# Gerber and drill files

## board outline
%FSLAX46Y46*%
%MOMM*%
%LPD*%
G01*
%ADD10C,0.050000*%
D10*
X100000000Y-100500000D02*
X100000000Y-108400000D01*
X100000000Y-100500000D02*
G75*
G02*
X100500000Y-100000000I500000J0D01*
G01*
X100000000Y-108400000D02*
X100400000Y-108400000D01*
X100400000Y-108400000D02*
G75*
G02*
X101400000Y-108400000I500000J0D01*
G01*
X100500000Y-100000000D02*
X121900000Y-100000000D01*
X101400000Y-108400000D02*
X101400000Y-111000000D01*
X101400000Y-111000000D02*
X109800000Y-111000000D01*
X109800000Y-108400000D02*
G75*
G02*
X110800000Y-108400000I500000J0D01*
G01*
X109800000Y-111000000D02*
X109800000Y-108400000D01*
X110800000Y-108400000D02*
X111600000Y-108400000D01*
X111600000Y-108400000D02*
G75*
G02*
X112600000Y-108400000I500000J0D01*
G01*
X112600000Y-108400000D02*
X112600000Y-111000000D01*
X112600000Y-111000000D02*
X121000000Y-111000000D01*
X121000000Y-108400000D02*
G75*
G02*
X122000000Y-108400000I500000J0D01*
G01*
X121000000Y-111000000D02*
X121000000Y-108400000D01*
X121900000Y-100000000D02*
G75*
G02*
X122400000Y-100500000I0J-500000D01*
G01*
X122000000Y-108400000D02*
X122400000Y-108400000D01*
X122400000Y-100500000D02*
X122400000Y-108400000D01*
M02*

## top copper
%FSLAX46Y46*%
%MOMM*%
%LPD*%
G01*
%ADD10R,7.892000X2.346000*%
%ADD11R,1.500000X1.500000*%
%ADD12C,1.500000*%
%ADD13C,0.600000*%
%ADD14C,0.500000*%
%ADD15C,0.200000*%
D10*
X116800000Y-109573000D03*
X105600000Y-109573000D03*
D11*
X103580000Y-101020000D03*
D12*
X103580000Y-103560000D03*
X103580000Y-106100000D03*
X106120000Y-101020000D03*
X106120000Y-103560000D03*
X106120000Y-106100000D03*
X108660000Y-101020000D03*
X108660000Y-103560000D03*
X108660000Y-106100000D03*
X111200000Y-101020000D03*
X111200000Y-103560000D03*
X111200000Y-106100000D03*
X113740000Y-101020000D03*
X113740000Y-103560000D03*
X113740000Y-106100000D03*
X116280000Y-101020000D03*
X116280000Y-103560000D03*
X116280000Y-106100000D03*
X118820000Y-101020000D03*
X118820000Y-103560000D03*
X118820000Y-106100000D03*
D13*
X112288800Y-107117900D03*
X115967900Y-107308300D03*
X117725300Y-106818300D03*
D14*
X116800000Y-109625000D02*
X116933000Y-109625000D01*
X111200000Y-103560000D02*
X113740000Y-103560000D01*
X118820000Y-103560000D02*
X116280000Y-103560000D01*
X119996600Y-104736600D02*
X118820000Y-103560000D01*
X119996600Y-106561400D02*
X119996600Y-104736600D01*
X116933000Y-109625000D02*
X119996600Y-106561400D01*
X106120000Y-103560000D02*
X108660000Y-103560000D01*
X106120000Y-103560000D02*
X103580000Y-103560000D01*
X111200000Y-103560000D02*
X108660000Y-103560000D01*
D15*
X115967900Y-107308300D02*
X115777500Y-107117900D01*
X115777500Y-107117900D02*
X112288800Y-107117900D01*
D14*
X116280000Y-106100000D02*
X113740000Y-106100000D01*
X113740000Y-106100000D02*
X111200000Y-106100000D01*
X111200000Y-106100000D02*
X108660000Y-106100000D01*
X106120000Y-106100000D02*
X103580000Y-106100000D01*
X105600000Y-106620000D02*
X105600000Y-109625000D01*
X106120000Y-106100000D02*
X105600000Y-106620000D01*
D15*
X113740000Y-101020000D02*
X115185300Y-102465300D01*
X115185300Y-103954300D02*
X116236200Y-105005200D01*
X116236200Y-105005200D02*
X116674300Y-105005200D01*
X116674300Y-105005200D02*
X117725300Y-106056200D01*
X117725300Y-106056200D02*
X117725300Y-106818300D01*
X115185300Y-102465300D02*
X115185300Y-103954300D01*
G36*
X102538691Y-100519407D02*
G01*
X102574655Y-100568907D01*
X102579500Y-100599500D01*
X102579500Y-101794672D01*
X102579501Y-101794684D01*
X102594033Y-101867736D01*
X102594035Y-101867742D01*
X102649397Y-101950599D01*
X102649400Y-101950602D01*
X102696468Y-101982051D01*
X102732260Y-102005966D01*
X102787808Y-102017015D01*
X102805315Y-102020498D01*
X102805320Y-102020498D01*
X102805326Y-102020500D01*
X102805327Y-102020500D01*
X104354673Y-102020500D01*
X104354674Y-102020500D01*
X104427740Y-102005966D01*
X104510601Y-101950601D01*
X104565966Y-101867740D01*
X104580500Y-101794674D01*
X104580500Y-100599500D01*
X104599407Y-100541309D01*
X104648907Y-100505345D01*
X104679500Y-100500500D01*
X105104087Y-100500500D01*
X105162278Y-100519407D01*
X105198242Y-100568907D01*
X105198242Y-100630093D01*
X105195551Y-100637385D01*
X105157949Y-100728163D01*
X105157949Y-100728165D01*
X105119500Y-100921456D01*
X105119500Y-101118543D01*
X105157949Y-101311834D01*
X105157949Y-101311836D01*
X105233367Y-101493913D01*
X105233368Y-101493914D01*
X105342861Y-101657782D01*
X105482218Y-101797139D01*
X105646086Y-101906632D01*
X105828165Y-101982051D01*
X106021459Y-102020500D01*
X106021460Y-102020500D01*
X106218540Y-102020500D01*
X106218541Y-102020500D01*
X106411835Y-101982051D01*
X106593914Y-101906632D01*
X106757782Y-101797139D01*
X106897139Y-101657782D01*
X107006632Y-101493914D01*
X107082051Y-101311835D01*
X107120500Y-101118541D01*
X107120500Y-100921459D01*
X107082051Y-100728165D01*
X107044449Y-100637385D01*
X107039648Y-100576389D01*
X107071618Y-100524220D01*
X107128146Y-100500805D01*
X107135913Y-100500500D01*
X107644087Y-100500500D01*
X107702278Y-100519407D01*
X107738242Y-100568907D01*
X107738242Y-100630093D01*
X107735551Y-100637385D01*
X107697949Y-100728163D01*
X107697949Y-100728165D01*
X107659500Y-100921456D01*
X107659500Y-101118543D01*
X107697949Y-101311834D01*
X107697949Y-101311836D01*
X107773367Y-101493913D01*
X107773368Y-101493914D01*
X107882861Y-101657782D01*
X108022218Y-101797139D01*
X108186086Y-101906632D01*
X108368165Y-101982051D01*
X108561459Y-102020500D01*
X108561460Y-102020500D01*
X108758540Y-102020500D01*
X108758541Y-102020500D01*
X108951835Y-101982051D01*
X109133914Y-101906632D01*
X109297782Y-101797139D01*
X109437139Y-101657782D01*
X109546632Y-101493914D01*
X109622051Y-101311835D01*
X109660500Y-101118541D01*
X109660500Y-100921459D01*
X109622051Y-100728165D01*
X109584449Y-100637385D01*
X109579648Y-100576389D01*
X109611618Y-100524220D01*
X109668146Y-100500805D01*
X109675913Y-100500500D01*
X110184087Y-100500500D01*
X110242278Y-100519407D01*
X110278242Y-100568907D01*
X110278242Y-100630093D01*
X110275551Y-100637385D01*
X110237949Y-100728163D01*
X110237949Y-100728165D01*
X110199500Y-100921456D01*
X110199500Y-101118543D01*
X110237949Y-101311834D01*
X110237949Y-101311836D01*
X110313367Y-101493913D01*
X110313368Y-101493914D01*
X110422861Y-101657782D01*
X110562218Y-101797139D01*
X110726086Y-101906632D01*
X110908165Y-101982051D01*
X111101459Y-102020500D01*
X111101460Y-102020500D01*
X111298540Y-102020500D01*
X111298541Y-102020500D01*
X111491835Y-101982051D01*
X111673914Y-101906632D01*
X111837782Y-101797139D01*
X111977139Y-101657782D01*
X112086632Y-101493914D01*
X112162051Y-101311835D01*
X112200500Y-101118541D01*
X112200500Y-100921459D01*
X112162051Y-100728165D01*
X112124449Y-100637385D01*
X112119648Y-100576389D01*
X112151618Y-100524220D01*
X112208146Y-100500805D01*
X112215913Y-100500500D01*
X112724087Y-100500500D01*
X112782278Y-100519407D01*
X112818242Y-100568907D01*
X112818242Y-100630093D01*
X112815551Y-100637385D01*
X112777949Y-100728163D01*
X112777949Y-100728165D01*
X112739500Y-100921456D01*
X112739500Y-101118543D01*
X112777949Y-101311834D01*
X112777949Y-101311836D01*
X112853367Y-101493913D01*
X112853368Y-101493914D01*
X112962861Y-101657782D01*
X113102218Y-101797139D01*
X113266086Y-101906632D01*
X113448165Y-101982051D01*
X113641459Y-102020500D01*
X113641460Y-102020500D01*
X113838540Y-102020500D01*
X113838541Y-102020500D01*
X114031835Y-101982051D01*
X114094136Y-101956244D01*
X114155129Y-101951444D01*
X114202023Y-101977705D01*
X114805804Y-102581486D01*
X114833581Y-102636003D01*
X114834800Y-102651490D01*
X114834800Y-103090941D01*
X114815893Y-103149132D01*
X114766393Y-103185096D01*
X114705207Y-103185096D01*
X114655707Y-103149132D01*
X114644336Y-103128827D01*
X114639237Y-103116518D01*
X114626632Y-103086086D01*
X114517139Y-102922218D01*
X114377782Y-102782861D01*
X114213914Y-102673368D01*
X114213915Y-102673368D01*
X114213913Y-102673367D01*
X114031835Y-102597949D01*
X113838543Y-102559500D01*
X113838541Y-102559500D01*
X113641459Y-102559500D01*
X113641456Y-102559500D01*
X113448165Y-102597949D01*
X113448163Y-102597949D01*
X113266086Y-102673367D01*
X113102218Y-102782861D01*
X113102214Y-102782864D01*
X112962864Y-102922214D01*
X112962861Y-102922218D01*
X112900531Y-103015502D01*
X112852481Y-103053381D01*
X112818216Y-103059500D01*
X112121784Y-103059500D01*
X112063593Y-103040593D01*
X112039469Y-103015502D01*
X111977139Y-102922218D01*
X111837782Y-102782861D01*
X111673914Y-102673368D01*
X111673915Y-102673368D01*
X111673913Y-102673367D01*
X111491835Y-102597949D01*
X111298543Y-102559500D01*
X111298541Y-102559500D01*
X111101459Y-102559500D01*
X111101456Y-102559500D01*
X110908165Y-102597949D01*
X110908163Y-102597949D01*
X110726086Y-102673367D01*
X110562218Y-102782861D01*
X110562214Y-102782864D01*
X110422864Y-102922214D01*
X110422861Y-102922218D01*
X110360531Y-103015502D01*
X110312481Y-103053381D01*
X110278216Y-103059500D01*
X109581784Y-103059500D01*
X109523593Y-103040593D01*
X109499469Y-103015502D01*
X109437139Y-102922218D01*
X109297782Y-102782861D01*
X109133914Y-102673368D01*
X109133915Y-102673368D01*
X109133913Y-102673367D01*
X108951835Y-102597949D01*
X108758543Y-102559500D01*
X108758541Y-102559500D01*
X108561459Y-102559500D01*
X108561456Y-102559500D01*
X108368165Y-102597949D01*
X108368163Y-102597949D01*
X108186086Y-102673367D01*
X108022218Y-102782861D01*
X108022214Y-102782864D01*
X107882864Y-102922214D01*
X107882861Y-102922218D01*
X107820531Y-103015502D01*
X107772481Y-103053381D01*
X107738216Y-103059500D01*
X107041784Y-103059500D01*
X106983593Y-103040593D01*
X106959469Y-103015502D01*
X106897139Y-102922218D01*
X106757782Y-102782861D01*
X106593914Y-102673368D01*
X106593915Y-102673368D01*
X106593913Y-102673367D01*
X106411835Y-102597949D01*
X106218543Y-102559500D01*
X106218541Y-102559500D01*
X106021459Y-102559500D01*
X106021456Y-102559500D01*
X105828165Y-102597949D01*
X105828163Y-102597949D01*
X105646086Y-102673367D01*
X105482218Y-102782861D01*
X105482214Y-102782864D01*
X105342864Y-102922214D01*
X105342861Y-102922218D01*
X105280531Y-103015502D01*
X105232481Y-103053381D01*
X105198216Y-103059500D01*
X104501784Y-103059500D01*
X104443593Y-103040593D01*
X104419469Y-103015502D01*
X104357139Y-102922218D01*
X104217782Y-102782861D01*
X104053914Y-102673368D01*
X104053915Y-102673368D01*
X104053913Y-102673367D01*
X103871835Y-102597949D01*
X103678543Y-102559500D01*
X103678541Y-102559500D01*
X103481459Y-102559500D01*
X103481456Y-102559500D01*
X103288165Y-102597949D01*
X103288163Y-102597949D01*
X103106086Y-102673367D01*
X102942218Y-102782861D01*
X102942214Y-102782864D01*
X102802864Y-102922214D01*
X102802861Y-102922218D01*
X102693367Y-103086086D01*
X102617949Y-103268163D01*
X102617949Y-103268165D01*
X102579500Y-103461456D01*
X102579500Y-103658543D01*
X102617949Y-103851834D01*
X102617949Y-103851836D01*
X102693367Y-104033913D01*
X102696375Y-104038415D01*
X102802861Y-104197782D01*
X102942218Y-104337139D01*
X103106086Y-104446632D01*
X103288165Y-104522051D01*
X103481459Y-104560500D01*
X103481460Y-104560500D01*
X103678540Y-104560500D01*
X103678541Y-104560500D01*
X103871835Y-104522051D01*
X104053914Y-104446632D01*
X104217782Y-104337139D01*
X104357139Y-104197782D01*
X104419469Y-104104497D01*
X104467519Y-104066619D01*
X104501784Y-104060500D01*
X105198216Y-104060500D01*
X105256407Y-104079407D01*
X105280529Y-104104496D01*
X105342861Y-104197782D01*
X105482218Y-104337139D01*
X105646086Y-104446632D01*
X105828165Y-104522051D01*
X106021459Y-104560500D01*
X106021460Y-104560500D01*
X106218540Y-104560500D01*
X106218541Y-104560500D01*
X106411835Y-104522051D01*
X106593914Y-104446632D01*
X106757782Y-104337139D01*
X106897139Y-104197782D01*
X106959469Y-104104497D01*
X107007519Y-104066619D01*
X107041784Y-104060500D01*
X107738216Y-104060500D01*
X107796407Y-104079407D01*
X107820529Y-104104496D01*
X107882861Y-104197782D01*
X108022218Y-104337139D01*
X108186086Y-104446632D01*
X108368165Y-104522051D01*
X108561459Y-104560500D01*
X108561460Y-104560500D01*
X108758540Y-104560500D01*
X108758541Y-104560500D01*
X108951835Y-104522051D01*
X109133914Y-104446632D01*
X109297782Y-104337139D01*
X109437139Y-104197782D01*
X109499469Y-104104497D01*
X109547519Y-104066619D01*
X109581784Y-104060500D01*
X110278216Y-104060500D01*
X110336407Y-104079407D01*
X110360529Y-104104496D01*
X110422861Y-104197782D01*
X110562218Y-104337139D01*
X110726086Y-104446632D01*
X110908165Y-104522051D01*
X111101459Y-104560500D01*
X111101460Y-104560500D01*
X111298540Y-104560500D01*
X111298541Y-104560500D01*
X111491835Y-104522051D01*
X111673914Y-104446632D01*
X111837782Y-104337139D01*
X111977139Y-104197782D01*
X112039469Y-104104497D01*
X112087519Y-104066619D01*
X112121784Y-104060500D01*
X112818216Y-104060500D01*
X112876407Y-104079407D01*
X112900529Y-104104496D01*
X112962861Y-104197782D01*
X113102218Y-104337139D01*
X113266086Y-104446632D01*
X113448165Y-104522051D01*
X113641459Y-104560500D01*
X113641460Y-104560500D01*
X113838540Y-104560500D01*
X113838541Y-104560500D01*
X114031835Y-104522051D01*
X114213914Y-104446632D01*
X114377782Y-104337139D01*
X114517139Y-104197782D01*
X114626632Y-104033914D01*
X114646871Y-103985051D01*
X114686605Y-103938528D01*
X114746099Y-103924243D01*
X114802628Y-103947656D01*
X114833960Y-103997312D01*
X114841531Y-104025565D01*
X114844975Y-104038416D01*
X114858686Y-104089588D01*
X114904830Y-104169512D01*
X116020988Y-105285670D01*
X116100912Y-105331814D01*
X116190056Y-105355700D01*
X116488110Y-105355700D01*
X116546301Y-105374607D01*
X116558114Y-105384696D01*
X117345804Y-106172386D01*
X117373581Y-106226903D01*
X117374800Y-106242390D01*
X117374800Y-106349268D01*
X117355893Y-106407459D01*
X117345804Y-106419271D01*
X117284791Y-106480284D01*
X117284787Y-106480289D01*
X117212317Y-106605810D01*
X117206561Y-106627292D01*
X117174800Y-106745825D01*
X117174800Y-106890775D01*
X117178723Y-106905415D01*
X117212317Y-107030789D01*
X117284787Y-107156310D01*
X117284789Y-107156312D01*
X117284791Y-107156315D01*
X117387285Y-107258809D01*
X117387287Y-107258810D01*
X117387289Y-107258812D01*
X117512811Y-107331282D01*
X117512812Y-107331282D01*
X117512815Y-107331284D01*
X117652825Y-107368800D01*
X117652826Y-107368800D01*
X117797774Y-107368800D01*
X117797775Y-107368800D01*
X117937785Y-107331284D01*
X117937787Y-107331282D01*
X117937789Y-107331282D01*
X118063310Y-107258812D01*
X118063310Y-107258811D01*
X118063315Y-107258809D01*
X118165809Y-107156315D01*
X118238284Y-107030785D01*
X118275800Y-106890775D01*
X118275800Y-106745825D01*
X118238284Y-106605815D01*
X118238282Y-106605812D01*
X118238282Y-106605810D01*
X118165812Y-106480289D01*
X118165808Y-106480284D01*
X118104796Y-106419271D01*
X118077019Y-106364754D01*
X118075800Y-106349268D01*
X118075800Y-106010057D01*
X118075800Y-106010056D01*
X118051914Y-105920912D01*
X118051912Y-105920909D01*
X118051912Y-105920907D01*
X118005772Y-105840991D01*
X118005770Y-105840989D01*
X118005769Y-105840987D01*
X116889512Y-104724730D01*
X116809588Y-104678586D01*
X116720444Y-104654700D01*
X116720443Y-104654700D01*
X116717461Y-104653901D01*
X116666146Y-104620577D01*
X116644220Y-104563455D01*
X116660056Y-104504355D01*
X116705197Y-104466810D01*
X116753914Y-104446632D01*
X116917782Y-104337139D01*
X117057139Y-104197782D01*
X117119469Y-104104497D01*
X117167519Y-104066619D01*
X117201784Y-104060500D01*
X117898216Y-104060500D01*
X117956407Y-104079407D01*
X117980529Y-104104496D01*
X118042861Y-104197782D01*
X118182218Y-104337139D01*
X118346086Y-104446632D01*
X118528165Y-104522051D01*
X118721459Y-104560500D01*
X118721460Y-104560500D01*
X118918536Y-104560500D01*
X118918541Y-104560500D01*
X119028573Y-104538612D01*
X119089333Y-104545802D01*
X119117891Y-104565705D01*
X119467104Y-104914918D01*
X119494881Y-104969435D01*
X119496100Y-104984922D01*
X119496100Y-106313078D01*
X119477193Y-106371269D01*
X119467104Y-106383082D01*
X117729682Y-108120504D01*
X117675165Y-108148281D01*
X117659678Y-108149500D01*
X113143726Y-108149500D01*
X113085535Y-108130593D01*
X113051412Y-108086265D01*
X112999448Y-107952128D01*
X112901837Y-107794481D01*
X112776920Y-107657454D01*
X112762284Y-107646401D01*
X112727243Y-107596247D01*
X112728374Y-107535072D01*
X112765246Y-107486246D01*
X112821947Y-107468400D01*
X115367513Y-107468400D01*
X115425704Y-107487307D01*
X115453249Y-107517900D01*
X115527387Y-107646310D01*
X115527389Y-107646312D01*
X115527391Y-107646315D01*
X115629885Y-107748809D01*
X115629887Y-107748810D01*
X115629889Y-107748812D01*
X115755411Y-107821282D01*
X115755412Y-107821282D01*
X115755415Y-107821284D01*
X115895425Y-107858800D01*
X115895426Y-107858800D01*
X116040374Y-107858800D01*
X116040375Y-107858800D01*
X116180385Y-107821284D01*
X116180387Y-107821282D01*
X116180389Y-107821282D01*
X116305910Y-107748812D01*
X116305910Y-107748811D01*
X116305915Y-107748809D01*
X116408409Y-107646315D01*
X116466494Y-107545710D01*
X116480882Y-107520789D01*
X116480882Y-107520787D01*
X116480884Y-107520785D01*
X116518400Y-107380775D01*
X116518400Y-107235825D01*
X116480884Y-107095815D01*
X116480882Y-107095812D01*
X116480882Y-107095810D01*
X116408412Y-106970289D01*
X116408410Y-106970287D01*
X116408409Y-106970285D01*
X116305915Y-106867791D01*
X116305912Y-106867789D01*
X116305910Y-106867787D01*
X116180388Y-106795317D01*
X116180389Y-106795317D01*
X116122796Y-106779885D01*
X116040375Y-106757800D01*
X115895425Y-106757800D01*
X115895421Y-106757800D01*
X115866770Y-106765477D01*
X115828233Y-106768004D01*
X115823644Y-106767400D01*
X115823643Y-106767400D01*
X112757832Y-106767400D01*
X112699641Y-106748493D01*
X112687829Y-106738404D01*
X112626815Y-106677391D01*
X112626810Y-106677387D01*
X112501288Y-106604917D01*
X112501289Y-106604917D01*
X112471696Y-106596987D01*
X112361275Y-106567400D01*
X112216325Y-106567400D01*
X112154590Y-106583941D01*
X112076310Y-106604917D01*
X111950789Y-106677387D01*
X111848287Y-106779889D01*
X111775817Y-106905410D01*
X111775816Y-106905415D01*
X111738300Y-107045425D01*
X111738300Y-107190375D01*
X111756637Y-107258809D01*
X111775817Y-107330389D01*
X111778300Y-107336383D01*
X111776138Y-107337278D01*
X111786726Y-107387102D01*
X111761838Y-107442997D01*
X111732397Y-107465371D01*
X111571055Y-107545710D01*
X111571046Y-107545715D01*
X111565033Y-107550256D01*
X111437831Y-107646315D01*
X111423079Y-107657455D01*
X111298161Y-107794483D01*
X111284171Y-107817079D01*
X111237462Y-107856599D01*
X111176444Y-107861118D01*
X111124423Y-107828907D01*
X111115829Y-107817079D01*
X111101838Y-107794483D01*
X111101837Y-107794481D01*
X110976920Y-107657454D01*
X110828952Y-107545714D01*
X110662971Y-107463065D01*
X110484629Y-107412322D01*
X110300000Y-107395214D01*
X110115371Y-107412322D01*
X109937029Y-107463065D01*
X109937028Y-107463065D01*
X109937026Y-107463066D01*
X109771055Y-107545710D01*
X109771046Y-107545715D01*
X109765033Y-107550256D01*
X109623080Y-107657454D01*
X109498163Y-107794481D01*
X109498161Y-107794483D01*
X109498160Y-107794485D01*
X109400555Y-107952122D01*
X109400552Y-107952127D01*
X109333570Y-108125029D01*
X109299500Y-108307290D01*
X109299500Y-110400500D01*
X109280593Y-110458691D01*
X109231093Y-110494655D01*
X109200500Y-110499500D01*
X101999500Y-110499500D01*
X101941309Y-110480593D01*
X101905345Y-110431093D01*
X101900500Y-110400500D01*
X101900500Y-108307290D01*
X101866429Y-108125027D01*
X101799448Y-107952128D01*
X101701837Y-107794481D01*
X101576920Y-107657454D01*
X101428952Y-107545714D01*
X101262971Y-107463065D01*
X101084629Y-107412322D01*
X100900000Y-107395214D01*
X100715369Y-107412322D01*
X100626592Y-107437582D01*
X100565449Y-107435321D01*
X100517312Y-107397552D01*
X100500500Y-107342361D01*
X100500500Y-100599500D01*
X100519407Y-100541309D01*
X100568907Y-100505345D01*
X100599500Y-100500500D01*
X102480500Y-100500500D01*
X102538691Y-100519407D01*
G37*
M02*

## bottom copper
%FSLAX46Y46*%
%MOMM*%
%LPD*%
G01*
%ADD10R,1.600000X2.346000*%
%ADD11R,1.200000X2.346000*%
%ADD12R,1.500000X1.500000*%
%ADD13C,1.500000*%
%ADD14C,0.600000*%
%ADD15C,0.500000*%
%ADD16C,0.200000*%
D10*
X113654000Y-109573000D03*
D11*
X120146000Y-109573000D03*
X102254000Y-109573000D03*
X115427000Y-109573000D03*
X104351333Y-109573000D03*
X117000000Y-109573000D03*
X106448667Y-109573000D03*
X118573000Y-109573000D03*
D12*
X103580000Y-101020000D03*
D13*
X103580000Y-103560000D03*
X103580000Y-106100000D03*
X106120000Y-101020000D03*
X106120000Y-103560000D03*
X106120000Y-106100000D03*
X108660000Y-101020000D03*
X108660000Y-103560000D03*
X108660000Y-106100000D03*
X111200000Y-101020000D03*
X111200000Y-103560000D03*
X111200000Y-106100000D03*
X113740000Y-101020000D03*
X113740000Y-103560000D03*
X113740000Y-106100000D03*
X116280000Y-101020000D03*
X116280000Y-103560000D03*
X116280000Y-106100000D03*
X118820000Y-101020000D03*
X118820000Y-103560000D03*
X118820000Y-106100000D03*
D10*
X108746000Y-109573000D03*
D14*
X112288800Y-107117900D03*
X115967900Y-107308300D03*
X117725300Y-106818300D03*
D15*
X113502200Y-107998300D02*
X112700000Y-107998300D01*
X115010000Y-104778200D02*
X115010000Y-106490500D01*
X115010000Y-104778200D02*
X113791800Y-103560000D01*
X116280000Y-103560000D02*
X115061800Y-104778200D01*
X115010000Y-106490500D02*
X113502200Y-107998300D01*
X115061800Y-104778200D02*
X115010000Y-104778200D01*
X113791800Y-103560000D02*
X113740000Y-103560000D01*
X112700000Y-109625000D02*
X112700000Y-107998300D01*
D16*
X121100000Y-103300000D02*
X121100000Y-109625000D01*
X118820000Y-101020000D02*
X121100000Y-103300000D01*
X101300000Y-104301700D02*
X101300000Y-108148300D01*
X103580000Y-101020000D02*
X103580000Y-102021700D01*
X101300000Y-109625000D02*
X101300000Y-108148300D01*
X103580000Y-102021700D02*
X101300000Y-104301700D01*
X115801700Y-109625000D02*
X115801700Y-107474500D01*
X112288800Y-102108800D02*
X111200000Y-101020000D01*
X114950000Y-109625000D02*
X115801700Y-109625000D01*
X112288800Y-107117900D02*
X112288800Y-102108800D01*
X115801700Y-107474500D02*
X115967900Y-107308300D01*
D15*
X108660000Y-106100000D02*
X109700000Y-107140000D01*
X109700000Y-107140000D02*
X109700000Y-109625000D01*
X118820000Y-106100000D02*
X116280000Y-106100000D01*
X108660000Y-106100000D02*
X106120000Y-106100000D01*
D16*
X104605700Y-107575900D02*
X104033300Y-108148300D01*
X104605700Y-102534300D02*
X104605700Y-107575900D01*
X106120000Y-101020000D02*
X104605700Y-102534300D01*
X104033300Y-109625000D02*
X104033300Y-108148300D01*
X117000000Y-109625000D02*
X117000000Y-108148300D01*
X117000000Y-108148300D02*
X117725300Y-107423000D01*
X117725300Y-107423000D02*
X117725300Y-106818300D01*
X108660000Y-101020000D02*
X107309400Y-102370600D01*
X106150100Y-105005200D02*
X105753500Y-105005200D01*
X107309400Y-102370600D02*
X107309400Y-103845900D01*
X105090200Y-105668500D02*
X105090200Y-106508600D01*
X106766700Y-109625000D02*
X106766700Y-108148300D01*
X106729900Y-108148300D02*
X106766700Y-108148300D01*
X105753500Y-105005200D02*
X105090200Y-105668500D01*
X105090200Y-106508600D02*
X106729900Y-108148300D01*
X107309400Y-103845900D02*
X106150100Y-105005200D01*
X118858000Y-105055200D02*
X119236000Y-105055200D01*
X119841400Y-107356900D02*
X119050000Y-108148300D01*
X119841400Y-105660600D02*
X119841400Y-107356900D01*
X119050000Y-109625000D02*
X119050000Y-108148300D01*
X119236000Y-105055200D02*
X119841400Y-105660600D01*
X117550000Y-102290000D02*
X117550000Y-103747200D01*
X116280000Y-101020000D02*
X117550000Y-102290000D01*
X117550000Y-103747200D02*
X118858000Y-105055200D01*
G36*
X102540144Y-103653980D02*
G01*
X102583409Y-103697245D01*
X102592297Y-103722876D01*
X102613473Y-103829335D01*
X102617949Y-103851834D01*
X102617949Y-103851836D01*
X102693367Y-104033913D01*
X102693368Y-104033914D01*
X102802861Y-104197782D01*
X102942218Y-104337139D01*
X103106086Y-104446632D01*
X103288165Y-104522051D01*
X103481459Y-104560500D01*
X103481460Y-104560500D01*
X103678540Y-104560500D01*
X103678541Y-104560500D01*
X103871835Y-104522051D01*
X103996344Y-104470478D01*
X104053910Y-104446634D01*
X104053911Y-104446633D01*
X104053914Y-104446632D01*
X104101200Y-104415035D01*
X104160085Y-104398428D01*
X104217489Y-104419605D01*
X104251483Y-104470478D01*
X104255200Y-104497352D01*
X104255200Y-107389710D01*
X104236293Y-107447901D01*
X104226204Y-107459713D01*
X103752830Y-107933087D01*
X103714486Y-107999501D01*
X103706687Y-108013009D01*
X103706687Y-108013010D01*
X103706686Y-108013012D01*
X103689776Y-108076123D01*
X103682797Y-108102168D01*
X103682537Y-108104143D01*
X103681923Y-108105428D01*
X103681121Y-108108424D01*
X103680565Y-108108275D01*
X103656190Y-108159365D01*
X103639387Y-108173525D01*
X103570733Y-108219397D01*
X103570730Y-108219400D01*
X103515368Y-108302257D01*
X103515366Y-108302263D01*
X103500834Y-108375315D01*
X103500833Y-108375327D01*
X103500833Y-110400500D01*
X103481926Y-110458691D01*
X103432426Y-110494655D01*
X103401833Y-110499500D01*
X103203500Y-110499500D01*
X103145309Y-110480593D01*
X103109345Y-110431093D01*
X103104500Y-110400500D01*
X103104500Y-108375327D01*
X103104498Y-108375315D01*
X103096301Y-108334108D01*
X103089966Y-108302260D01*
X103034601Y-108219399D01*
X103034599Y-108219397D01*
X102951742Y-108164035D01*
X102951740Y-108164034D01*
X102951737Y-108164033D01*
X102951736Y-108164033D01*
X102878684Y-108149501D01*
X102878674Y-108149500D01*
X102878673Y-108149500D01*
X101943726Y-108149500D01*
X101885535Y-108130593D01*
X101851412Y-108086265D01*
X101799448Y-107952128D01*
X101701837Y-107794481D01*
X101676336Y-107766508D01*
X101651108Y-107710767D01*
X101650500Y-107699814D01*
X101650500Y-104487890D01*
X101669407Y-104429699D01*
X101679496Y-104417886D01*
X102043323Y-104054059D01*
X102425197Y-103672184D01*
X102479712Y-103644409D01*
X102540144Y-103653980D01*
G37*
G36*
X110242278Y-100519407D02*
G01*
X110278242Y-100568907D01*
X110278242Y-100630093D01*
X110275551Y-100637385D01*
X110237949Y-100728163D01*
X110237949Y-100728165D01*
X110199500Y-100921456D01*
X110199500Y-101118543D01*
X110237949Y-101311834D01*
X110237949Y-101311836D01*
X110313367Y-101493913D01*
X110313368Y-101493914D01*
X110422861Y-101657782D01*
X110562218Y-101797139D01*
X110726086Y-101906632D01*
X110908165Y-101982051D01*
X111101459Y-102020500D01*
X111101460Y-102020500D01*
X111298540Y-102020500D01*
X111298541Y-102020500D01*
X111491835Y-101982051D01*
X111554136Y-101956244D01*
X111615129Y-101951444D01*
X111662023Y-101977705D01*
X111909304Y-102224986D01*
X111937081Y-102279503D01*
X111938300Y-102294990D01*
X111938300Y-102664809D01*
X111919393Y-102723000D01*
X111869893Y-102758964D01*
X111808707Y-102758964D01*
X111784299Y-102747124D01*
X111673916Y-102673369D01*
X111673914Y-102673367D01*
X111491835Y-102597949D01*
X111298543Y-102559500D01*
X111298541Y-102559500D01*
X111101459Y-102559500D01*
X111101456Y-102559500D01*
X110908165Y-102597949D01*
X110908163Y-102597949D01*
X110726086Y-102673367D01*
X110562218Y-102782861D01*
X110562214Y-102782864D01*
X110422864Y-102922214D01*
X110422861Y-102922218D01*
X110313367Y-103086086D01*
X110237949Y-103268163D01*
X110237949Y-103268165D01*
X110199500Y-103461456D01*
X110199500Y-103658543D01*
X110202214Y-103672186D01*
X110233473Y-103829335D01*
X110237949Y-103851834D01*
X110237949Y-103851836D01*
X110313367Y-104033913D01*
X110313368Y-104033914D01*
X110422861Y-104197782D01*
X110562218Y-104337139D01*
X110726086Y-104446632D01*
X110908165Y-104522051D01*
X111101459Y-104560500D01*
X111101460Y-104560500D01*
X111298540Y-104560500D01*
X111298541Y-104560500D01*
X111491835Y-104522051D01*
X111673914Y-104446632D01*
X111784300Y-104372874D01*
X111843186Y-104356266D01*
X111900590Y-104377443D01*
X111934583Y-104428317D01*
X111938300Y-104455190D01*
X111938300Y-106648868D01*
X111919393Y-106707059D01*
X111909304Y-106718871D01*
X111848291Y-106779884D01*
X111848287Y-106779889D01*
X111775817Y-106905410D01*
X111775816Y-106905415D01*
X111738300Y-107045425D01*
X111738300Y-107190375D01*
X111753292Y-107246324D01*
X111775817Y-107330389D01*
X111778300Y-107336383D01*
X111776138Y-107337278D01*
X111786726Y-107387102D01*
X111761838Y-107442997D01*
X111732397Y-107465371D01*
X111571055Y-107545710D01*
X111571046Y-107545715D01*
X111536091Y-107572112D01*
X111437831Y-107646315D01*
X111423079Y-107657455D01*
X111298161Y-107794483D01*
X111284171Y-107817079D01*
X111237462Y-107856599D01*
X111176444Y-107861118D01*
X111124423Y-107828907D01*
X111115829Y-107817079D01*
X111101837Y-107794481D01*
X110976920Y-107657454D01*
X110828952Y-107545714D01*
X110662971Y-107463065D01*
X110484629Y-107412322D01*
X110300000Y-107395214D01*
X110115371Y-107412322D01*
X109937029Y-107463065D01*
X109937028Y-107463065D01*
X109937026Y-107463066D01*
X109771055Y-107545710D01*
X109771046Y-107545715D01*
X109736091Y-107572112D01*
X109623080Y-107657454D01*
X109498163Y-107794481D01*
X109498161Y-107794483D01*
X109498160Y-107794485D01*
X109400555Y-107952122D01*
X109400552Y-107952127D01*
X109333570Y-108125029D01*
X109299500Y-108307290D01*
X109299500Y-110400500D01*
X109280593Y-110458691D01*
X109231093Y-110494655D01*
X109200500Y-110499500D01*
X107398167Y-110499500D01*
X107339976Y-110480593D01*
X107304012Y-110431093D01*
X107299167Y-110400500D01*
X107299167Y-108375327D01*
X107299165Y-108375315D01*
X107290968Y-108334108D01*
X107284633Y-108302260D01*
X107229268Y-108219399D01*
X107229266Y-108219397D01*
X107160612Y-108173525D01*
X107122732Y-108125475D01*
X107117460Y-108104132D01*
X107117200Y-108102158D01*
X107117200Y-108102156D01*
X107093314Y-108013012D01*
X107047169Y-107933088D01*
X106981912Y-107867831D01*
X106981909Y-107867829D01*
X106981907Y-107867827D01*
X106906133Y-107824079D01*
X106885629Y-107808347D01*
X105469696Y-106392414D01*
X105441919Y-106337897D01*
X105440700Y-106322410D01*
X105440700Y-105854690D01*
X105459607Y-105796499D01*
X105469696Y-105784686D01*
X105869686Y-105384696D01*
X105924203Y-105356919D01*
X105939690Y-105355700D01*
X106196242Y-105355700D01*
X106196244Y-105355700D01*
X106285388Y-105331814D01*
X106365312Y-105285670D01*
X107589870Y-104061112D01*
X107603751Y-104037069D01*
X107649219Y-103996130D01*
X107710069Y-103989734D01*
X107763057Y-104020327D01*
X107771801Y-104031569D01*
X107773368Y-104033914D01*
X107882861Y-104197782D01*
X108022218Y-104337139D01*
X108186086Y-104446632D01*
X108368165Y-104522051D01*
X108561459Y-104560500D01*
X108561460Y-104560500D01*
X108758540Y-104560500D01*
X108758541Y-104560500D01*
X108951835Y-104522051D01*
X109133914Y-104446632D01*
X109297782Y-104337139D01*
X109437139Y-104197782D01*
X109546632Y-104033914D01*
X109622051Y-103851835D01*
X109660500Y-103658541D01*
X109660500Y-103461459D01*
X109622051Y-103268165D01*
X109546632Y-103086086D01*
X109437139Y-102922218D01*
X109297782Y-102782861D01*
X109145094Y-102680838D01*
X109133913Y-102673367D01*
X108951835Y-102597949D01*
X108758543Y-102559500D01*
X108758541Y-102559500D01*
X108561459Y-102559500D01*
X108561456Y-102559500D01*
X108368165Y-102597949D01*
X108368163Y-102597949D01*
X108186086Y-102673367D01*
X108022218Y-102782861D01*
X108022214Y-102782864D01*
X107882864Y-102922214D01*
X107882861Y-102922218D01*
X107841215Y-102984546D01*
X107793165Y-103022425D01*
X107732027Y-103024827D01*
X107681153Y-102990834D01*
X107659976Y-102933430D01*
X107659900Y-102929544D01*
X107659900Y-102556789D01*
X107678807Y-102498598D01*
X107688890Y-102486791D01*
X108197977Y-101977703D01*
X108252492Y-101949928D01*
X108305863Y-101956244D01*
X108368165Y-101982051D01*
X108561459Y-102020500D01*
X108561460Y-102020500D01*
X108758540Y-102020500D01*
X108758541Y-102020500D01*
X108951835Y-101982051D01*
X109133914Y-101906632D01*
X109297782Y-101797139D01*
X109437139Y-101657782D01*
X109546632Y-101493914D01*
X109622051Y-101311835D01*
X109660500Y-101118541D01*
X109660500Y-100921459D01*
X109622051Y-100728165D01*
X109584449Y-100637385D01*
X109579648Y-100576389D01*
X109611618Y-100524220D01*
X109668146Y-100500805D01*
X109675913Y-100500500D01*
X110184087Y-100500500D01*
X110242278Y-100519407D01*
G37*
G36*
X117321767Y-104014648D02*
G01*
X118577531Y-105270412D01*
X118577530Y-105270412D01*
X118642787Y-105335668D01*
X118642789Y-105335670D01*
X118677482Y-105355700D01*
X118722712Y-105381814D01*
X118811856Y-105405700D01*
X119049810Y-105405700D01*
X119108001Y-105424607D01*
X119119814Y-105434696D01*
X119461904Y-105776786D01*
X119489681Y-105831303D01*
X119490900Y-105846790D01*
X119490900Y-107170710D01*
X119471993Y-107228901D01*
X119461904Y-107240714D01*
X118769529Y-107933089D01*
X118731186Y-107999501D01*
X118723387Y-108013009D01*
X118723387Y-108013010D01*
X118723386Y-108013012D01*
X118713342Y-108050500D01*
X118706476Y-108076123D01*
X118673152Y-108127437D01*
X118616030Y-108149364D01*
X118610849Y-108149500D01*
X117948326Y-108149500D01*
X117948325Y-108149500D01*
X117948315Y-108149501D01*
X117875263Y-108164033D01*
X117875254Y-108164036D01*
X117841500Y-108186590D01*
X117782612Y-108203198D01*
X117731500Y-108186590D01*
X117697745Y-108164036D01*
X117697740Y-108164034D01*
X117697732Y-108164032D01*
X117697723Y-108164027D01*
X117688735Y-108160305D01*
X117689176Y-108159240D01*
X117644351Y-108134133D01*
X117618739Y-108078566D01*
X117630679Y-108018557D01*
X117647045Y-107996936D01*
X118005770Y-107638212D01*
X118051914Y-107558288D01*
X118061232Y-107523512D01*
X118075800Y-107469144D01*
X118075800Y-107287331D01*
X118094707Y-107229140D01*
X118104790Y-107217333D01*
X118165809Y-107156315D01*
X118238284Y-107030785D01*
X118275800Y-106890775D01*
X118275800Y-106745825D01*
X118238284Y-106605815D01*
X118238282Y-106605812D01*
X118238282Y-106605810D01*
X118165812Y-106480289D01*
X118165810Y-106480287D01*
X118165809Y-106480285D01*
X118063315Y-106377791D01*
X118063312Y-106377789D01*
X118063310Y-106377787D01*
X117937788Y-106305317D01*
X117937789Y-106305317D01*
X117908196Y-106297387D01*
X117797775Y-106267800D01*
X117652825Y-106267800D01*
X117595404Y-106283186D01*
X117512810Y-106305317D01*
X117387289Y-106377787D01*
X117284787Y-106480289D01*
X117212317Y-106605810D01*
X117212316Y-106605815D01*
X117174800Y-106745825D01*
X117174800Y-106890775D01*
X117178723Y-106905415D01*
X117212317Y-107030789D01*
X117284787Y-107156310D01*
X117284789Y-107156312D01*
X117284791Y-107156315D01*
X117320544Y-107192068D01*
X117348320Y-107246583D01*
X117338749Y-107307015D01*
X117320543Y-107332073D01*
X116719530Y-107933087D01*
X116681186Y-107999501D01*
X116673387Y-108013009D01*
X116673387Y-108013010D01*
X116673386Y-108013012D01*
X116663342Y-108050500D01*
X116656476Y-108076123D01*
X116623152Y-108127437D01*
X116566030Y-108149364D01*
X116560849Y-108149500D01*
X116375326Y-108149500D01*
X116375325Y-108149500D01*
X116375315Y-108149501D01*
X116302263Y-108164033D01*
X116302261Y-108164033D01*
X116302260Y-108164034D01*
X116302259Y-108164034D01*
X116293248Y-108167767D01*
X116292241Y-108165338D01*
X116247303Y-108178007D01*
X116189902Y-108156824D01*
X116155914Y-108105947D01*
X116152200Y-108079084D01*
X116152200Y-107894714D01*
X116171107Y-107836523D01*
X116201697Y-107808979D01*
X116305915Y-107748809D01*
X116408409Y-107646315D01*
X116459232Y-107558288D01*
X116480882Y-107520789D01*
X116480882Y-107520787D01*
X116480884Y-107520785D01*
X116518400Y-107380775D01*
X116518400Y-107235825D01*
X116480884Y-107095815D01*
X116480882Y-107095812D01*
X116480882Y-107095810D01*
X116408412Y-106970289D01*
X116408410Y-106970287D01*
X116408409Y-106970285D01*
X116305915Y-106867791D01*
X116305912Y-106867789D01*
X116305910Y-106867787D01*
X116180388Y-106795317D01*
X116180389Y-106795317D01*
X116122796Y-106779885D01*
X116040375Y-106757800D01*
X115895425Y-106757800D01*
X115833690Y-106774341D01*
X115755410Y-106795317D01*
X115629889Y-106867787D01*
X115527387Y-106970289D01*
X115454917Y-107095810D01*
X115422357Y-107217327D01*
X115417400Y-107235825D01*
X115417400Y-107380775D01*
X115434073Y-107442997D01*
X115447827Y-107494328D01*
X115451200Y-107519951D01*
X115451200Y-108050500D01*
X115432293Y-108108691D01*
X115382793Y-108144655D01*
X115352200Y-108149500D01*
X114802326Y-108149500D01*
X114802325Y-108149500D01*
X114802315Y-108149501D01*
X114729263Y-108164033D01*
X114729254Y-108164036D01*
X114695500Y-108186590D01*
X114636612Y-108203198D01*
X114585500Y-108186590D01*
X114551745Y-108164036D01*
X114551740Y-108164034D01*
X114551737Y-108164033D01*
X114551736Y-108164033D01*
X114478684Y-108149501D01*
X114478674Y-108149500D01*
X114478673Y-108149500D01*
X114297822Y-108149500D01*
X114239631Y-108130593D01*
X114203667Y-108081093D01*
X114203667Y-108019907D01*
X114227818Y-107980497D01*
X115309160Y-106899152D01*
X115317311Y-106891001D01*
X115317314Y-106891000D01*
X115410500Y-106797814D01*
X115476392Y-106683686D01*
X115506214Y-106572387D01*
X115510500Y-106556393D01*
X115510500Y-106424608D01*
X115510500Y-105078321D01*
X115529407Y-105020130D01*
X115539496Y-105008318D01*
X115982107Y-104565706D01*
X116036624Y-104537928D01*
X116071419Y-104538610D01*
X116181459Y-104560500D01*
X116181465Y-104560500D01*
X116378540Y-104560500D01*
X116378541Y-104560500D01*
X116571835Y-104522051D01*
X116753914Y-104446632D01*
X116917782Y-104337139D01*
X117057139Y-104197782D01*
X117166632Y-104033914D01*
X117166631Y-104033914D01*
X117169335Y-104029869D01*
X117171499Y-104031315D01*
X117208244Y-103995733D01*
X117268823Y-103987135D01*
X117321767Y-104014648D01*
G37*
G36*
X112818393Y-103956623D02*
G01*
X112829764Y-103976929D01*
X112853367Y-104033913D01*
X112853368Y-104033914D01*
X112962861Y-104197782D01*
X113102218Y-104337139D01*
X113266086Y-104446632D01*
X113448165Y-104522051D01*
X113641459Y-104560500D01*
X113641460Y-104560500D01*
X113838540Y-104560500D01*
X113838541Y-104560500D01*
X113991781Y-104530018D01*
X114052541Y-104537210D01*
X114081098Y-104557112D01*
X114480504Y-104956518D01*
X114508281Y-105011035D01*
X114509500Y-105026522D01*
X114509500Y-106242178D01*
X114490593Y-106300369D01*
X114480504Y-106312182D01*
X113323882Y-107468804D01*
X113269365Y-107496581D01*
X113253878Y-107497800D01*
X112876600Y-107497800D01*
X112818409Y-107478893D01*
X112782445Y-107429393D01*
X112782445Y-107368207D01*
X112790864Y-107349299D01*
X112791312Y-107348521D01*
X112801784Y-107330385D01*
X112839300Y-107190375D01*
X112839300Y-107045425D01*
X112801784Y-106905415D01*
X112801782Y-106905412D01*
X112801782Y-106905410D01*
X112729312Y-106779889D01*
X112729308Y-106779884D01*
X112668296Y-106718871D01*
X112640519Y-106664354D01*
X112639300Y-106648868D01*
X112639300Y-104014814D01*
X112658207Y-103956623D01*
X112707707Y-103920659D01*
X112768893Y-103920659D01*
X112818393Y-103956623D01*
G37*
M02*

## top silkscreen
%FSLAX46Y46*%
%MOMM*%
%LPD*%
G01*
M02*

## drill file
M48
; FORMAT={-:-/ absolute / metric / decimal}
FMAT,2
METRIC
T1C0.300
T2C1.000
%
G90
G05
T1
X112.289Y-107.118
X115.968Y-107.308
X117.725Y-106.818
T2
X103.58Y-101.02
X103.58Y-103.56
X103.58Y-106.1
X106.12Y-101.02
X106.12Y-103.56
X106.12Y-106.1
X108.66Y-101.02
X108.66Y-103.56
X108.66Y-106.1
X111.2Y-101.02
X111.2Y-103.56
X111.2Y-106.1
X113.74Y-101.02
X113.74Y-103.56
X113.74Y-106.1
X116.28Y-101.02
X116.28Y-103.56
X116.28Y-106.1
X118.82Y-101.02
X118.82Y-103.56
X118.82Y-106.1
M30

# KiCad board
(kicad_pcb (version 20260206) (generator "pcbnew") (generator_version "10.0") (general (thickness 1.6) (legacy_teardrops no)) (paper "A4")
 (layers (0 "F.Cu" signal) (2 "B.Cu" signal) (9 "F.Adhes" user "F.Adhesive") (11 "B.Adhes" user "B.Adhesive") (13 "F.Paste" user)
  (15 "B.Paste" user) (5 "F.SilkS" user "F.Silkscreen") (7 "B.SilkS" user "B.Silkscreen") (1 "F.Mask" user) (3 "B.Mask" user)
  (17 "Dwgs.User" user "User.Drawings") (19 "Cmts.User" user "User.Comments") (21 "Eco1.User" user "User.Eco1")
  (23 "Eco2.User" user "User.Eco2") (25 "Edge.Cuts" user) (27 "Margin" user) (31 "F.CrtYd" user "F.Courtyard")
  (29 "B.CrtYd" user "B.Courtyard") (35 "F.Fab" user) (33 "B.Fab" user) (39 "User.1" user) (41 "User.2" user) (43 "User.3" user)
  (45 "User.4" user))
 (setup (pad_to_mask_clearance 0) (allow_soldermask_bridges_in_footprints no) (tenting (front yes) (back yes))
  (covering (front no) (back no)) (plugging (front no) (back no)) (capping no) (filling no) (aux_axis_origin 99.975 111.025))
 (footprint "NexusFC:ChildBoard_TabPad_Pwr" (layer "F.Cu") (at 113.654 108.4)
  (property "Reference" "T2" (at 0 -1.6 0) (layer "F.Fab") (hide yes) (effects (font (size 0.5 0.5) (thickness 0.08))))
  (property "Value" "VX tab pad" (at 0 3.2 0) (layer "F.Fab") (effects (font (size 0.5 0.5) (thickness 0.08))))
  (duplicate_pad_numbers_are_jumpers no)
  (pad "1" smd rect (at 0 1.173) (size 1.6 2.346) (layers "B.Cu" "B.Mask") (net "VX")))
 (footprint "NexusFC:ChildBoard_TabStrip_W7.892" (layer "F.Cu") (at 116.8 108.4)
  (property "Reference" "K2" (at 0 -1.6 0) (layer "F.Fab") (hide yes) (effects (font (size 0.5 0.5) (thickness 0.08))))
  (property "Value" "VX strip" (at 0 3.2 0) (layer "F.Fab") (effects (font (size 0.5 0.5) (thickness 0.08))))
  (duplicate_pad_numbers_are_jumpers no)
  (pad "1" smd rect (at 0 1.173) (size 7.892 2.346) (layers "F.Cu" "F.Mask") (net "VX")))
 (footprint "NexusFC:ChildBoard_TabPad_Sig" (layer "F.Cu") (at 120.146 108.4)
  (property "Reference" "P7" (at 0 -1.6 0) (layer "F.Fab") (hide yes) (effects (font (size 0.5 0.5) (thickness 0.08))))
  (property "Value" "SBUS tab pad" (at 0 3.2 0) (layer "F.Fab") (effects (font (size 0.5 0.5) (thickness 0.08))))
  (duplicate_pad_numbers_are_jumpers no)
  (pad "1" smd rect (at 0 1.173) (size 1.2 2.346) (layers "B.Cu" "B.Mask") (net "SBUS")))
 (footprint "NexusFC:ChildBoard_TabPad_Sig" (layer "F.Cu") (at 102.254 108.4)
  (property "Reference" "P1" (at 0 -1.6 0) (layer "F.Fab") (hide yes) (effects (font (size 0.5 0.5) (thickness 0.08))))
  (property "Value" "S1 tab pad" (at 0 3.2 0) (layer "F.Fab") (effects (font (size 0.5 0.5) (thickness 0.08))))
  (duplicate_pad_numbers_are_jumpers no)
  (pad "1" smd rect (at 0 1.173) (size 1.2 2.346) (layers "B.Cu" "B.Mask") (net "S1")))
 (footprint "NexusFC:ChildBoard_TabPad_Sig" (layer "F.Cu") (at 115.427 108.4)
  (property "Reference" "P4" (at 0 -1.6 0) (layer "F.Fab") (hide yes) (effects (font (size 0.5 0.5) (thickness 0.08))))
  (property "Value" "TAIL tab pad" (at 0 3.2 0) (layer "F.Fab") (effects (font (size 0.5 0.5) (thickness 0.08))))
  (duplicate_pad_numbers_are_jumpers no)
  (pad "1" smd rect (at 0 1.173) (size 1.2 2.346) (layers "B.Cu" "B.Mask") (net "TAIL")))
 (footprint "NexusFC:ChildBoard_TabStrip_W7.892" (layer "F.Cu") (at 105.6 108.4)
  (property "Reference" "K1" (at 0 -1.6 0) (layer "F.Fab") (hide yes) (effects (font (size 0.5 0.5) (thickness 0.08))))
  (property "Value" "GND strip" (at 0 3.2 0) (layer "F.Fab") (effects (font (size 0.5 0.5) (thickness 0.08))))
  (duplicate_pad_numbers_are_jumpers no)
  (pad "1" smd rect (at 0 1.173) (size 7.892 2.346) (layers "F.Cu" "F.Mask") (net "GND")))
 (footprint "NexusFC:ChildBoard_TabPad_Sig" (layer "F.Cu") (at 104.351333 108.4)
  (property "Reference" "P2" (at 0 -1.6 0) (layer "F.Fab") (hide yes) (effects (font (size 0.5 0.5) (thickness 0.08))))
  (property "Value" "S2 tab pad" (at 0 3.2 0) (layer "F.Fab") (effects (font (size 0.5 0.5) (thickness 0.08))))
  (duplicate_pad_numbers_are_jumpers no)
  (pad "1" smd rect (at 0 1.173) (size 1.2 2.346) (layers "B.Cu" "B.Mask") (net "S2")))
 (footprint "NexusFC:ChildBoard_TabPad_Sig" (layer "F.Cu") (at 117 108.4)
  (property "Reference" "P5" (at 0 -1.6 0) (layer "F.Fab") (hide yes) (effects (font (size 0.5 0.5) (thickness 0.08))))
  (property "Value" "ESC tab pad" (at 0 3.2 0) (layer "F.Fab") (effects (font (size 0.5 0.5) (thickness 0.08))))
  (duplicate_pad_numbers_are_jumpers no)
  (pad "1" smd rect (at 0 1.173) (size 1.2 2.346) (layers "B.Cu" "B.Mask") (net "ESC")))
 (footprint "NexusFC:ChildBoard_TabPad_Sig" (layer "F.Cu") (at 106.448667 108.4)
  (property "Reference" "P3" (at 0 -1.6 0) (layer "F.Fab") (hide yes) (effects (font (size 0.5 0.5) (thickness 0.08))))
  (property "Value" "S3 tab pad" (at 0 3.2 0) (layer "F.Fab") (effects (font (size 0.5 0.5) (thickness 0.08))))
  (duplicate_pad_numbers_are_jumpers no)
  (pad "1" smd rect (at 0 1.173) (size 1.2 2.346) (layers "B.Cu" "B.Mask") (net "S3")))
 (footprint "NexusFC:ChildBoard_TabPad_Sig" (layer "F.Cu") (at 118.573 108.4)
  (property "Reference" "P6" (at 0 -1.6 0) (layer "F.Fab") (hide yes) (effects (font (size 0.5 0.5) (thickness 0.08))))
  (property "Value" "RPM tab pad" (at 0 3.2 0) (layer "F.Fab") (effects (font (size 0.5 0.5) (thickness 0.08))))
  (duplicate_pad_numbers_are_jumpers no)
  (pad "1" smd rect (at 0 1.173) (size 1.2 2.346) (layers "B.Cu" "B.Mask") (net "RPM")))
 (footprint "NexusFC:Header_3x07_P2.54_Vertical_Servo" (layer "F.Cu") (at 111.2 103.56)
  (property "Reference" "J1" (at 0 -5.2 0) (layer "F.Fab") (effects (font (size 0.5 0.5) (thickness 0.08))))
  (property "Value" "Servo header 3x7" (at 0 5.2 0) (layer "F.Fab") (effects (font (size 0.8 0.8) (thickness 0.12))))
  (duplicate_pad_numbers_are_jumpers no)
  (pad "1" thru_hole rect (at -7.62 -2.54) (size 1.5 1.5) (drill 1) (layers "*.Cu" "*.Mask") (remove_unused_layers no) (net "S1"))
  (pad "2" thru_hole circle (at -7.62 0) (size 1.5 1.5) (drill 1) (layers "*.Cu" "*.Mask") (remove_unused_layers no) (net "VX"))
  (pad "3" thru_hole circle (at -7.62 2.54) (size 1.5 1.5) (drill 1) (layers "*.Cu" "*.Mask") (remove_unused_layers no) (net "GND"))
  (pad "4" thru_hole circle (at -5.08 -2.54) (size 1.5 1.5) (drill 1) (layers "*.Cu" "*.Mask") (remove_unused_layers no) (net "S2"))
  (pad "5" thru_hole circle (at -5.08 0) (size 1.5 1.5) (drill 1) (layers "*.Cu" "*.Mask") (remove_unused_layers no) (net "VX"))
  (pad "6" thru_hole circle (at -5.08 2.54) (size 1.5 1.5) (drill 1) (layers "*.Cu" "*.Mask") (remove_unused_layers no) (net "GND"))
  (pad "7" thru_hole circle (at -2.54 -2.54) (size 1.5 1.5) (drill 1) (layers "*.Cu" "*.Mask") (remove_unused_layers no) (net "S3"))
  (pad "8" thru_hole circle (at -2.54 0) (size 1.5 1.5) (drill 1) (layers "*.Cu" "*.Mask") (remove_unused_layers no) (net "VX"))
  (pad "9" thru_hole circle (at -2.54 2.54) (size 1.5 1.5) (drill 1) (layers "*.Cu" "*.Mask") (remove_unused_layers no) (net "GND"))
  (pad "10" thru_hole circle (at 0 -2.54) (size 1.5 1.5) (drill 1) (layers "*.Cu" "*.Mask") (remove_unused_layers no) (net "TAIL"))
  (pad "11" thru_hole circle (at 0 0) (size 1.5 1.5) (drill 1) (layers "*.Cu" "*.Mask") (remove_unused_layers no) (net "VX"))
  (pad "12" thru_hole circle (at 0 2.54) (size 1.5 1.5) (drill 1) (layers "*.Cu" "*.Mask") (remove_unused_layers no) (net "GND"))
  (pad "13" thru_hole circle (at 2.54 -2.54) (size 1.5 1.5) (drill 1) (layers "*.Cu" "*.Mask") (remove_unused_layers no) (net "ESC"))
  (pad "14" thru_hole circle (at 2.54 0) (size 1.5 1.5) (drill 1) (layers "*.Cu" "*.Mask") (remove_unused_layers no) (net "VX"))
  (pad "15" thru_hole circle (at 2.54 2.54) (size 1.5 1.5) (drill 1) (layers "*.Cu" "*.Mask") (remove_unused_layers no) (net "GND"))
  (pad "16" thru_hole circle (at 5.08 -2.54) (size 1.5 1.5) (drill 1) (layers "*.Cu" "*.Mask") (remove_unused_layers no) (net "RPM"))
  (pad "17" thru_hole circle (at 5.08 0) (size 1.5 1.5) (drill 1) (layers "*.Cu" "*.Mask") (remove_unused_layers no) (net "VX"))
  (pad "18" thru_hole circle (at 5.08 2.54) (size 1.5 1.5) (drill 1) (layers "*.Cu" "*.Mask") (remove_unused_layers no) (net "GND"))
  (pad "19" thru_hole circle (at 7.62 -2.54) (size 1.5 1.5) (drill 1) (layers "*.Cu" "*.Mask") (remove_unused_layers no) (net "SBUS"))
  (pad "20" thru_hole circle (at 7.62 0) (size 1.5 1.5) (drill 1) (layers "*.Cu" "*.Mask") (remove_unused_layers no) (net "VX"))
  (pad "21" thru_hole circle (at 7.62 2.54) (size 1.5 1.5) (drill 1) (layers "*.Cu" "*.Mask") (remove_unused_layers no) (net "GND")))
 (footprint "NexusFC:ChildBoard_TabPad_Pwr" (layer "F.Cu") (at 108.746 108.4)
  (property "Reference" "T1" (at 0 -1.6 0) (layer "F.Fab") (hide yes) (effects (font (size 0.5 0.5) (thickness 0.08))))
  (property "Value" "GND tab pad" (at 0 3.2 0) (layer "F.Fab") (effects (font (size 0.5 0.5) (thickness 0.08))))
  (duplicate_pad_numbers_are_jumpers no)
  (pad "1" smd rect (at 0 1.173) (size 1.6 2.346) (layers "B.Cu" "B.Mask") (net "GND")))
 (gr_line (start 100 100.5) (end 100 108.4) (stroke (width 0.05) (type default)) (layer "Edge.Cuts"))
 (gr_arc (start 100 100.5) (mid 100.146447 100.146447) (end 100.5 100) (stroke (width 0.05) (type default)) (layer "Edge.Cuts"))
 (gr_line (start 100 108.4) (end 100.4 108.4) (stroke (width 0.05) (type solid)) (layer "Edge.Cuts"))
 (gr_arc (start 100.4 108.4) (mid 100.9 107.9) (end 101.4 108.4) (stroke (width 0.05) (type solid)) (layer "Edge.Cuts"))
 (gr_line (start 100.5 100) (end 121.9 100) (stroke (width 0.05) (type default)) (layer "Edge.Cuts"))
 (gr_line (start 101.4 108.4) (end 101.4 111) (stroke (width 0.05) (type solid)) (layer "Edge.Cuts"))
 (gr_line (start 101.4 111) (end 109.8 111) (stroke (width 0.05) (type solid)) (layer "Edge.Cuts"))
 (gr_arc (start 109.8 108.4) (mid 110.3 107.9) (end 110.8 108.4) (stroke (width 0.05) (type solid)) (layer "Edge.Cuts"))
 (gr_line (start 109.8 111) (end 109.8 108.4) (stroke (width 0.05) (type solid)) (layer "Edge.Cuts"))
 (gr_line (start 110.8 108.4) (end 111.6 108.4) (stroke (width 0.05) (type solid)) (layer "Edge.Cuts"))
 (gr_arc (start 111.6 108.4) (mid 112.1 107.9) (end 112.6 108.4) (stroke (width 0.05) (type solid)) (layer "Edge.Cuts"))
 (gr_line (start 112.6 108.4) (end 112.6 111) (stroke (width 0.05) (type solid)) (layer "Edge.Cuts"))
 (gr_line (start 112.6 111) (end 121 111) (stroke (width 0.05) (type solid)) (layer "Edge.Cuts"))
 (gr_arc (start 121 108.4) (mid 121.5 107.9) (end 122 108.4) (stroke (width 0.05) (type solid)) (layer "Edge.Cuts"))
 (gr_line (start 121 111) (end 121 108.4) (stroke (width 0.05) (type solid)) (layer "Edge.Cuts"))
 (gr_arc (start 121.9 100) (mid 122.253553 100.146447) (end 122.4 100.5) (stroke (width 0.05) (type default)) (layer "Edge.Cuts"))
 (gr_line (start 122 108.4) (end 122.4 108.4) (stroke (width 0.05) (type solid)) (layer "Edge.Cuts"))
 (gr_line (start 122.4 100.5) (end 122.4 108.4) (stroke (width 0.05) (type default)) (layer "Edge.Cuts"))
 (segment (start 116.8 109.625) (end 116.933 109.625) (width 0.5) (layer "F.Cu") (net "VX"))
 (segment (start 111.2 103.56) (end 113.74 103.56) (width 0.5) (layer "F.Cu") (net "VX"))
 (segment (start 118.82 103.56) (end 116.28 103.56) (width 0.5) (layer "F.Cu") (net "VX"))
 (segment (start 119.9966 104.7366) (end 118.82 103.56) (width 0.5) (layer "F.Cu") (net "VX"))
 (segment (start 119.9966 106.5614) (end 119.9966 104.7366) (width 0.5) (layer "F.Cu") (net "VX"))
 (segment (start 116.933 109.625) (end 119.9966 106.5614) (width 0.5) (layer "F.Cu") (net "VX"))
 (segment (start 106.12 103.56) (end 108.66 103.56) (width 0.5) (layer "F.Cu") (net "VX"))
 (segment (start 106.12 103.56) (end 103.58 103.56) (width 0.5) (layer "F.Cu") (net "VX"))
 (segment (start 111.2 103.56) (end 108.66 103.56) (width 0.5) (layer "F.Cu") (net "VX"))
 (segment (start 113.5022 107.9983) (end 112.7 107.9983) (width 0.5) (layer "B.Cu") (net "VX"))
 (segment (start 115.01 104.7782) (end 115.01 106.4905) (width 0.5) (layer "B.Cu") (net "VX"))
 (segment (start 115.01 104.7782) (end 113.7918 103.56) (width 0.5) (layer "B.Cu") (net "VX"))
 (segment (start 116.28 103.56) (end 115.0618 104.7782) (width 0.5) (layer "B.Cu") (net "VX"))
 (segment (start 115.01 106.4905) (end 113.5022 107.9983) (width 0.5) (layer "B.Cu") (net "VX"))
 (segment (start 115.0618 104.7782) (end 115.01 104.7782) (width 0.5) (layer "B.Cu") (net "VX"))
 (segment (start 113.7918 103.56) (end 113.74 103.56) (width 0.5) (layer "B.Cu") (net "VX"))
 (segment (start 112.7 109.625) (end 112.7 107.9983) (width 0.5) (layer "B.Cu") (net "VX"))
 (segment (start 121.1 103.3) (end 121.1 109.625) (width 0.2) (layer "B.Cu") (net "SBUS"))
 (segment (start 118.82 101.02) (end 121.1 103.3) (width 0.2) (layer "B.Cu") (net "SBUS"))
 (segment (start 101.3 104.3017) (end 101.3 108.1483) (width 0.2) (layer "B.Cu") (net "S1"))
 (segment (start 103.58 101.02) (end 103.58 102.0217) (width 0.2) (layer "B.Cu") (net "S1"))
 (segment (start 101.3 109.625) (end 101.3 108.1483) (width 0.2) (layer "B.Cu") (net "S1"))
 (segment (start 103.58 102.0217) (end 101.3 104.3017) (width 0.2) (layer "B.Cu") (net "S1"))
 (segment (start 115.9679 107.3083) (end 115.7775 107.1179) (width 0.2) (layer "F.Cu") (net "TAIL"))
 (segment (start 115.7775 107.1179) (end 112.2888 107.1179) (width 0.2) (layer "F.Cu") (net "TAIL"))
 (via (at 112.2888 107.1179) (size 0.6) (drill 0.3) (layers "F.Cu" "B.Cu") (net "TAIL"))
 (via (at 115.9679 107.3083) (size 0.6) (drill 0.3) (layers "F.Cu" "B.Cu") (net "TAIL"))
 (segment (start 115.8017 109.625) (end 115.8017 107.4745) (width 0.2) (layer "B.Cu") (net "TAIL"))
 (segment (start 112.2888 102.1088) (end 111.2 101.02) (width 0.2) (layer "B.Cu") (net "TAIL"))
 (segment (start 114.95 109.625) (end 115.8017 109.625) (width 0.2) (layer "B.Cu") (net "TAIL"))
 (segment (start 112.2888 107.1179) (end 112.2888 102.1088) (width 0.2) (layer "B.Cu") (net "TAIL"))
 (segment (start 115.8017 107.4745) (end 115.9679 107.3083) (width 0.2) (layer "B.Cu") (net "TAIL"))
 (segment (start 116.28 106.1) (end 113.74 106.1) (width 0.5) (layer "F.Cu") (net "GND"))
 (segment (start 113.74 106.1) (end 111.2 106.1) (width 0.5) (layer "F.Cu") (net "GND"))
 (segment (start 111.2 106.1) (end 108.66 106.1) (width 0.5) (layer "F.Cu") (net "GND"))
 (segment (start 106.12 106.1) (end 103.58 106.1) (width 0.5) (layer "F.Cu") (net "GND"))
 (segment (start 105.6 106.62) (end 105.6 109.625) (width 0.5) (layer "F.Cu") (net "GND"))
 (segment (start 106.12 106.1) (end 105.6 106.62) (width 0.5) (layer "F.Cu") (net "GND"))
 (segment (start 108.66 106.1) (end 109.7 107.14) (width 0.5) (layer "B.Cu") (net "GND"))
 (segment (start 109.7 107.14) (end 109.7 109.625) (width 0.5) (layer "B.Cu") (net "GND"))
 (segment (start 118.82 106.1) (end 116.28 106.1) (width 0.5) (layer "B.Cu") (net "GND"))
 (segment (start 108.66 106.1) (end 106.12 106.1) (width 0.5) (layer "B.Cu") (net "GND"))
 (segment (start 104.6057 107.5759) (end 104.0333 108.1483) (width 0.2) (layer "B.Cu") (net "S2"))
 (segment (start 104.6057 102.5343) (end 104.6057 107.5759) (width 0.2) (layer "B.Cu") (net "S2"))
 (segment (start 106.12 101.02) (end 104.6057 102.5343) (width 0.2) (layer "B.Cu") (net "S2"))
 (segment (start 104.0333 109.625) (end 104.0333 108.1483) (width 0.2) (layer "B.Cu") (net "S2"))
 (segment (start 113.74 101.02) (end 115.1853 102.4653) (width 0.2) (layer "F.Cu") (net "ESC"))
 (segment (start 115.1853 103.9543) (end 116.2362 105.0052) (width 0.2) (layer "F.Cu") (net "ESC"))
 (segment (start 116.2362 105.0052) (end 116.6743 105.0052) (width 0.2) (layer "F.Cu") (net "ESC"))
 (segment (start 116.6743 105.0052) (end 117.7253 106.0562) (width 0.2) (layer "F.Cu") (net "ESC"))
 (segment (start 117.7253 106.0562) (end 117.7253 106.8183) (width 0.2) (layer "F.Cu") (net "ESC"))
 (segment (start 115.1853 102.4653) (end 115.1853 103.9543) (width 0.2) (layer "F.Cu") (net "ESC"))
 (via (at 117.7253 106.8183) (size 0.6) (drill 0.3) (layers "F.Cu" "B.Cu") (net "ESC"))
 (segment (start 117 109.625) (end 117 108.1483) (width 0.2) (layer "B.Cu") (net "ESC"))
 (segment (start 117 108.1483) (end 117.7253 107.423) (width 0.2) (layer "B.Cu") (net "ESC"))
 (segment (start 117.7253 107.423) (end 117.7253 106.8183) (width 0.2) (layer "B.Cu") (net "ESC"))
 (segment (start 108.66 101.02) (end 107.3094 102.3706) (width 0.2) (layer "B.Cu") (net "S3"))
 (segment (start 106.1501 105.0052) (end 105.7535 105.0052) (width 0.2) (layer "B.Cu") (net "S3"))
 (segment (start 107.3094 102.3706) (end 107.3094 103.8459) (width 0.2) (layer "B.Cu") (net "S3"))
 (segment (start 105.0902 105.6685) (end 105.0902 106.5086) (width 0.2) (layer "B.Cu") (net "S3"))
 (segment (start 106.7667 109.625) (end 106.7667 108.1483) (width 0.2) (layer "B.Cu") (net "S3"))
 (segment (start 106.7299 108.1483) (end 106.7667 108.1483) (width 0.2) (layer "B.Cu") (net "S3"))
 (segment (start 105.7535 105.0052) (end 105.0902 105.6685) (width 0.2) (layer "B.Cu") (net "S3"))
 (segment (start 105.0902 106.5086) (end 106.7299 108.1483) (width 0.2) (layer "B.Cu") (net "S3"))
 (segment (start 107.3094 103.8459) (end 106.1501 105.0052) (width 0.2) (layer "B.Cu") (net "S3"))
 (segment (start 118.858 105.0552) (end 119.236 105.0552) (width 0.2) (layer "B.Cu") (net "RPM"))
 (segment (start 119.8414 107.3569) (end 119.05 108.1483) (width 0.2) (layer "B.Cu") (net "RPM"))
 (segment (start 119.8414 105.6606) (end 119.8414 107.3569) (width 0.2) (layer "B.Cu") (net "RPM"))
 (segment (start 119.05 109.625) (end 119.05 108.1483) (width 0.2) (layer "B.Cu") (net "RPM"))
 (segment (start 119.236 105.0552) (end 119.8414 105.6606) (width 0.2) (layer "B.Cu") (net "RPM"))
 (segment (start 117.55 102.29) (end 117.55 103.7472) (width 0.2) (layer "B.Cu") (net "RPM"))
 (segment (start 116.28 101.02) (end 117.55 102.29) (width 0.2) (layer "B.Cu") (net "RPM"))
 (segment (start 117.55 103.7472) (end 118.858 105.0552) (width 0.2) (layer "B.Cu") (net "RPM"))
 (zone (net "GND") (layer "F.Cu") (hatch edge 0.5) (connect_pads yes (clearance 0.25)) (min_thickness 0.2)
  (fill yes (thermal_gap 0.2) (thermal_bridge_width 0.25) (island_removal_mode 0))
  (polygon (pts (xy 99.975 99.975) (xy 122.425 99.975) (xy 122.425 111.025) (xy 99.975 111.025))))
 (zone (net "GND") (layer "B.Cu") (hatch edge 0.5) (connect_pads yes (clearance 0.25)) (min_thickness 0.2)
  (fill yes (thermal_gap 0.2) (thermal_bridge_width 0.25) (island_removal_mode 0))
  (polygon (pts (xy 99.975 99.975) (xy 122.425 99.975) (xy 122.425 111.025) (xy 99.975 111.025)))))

